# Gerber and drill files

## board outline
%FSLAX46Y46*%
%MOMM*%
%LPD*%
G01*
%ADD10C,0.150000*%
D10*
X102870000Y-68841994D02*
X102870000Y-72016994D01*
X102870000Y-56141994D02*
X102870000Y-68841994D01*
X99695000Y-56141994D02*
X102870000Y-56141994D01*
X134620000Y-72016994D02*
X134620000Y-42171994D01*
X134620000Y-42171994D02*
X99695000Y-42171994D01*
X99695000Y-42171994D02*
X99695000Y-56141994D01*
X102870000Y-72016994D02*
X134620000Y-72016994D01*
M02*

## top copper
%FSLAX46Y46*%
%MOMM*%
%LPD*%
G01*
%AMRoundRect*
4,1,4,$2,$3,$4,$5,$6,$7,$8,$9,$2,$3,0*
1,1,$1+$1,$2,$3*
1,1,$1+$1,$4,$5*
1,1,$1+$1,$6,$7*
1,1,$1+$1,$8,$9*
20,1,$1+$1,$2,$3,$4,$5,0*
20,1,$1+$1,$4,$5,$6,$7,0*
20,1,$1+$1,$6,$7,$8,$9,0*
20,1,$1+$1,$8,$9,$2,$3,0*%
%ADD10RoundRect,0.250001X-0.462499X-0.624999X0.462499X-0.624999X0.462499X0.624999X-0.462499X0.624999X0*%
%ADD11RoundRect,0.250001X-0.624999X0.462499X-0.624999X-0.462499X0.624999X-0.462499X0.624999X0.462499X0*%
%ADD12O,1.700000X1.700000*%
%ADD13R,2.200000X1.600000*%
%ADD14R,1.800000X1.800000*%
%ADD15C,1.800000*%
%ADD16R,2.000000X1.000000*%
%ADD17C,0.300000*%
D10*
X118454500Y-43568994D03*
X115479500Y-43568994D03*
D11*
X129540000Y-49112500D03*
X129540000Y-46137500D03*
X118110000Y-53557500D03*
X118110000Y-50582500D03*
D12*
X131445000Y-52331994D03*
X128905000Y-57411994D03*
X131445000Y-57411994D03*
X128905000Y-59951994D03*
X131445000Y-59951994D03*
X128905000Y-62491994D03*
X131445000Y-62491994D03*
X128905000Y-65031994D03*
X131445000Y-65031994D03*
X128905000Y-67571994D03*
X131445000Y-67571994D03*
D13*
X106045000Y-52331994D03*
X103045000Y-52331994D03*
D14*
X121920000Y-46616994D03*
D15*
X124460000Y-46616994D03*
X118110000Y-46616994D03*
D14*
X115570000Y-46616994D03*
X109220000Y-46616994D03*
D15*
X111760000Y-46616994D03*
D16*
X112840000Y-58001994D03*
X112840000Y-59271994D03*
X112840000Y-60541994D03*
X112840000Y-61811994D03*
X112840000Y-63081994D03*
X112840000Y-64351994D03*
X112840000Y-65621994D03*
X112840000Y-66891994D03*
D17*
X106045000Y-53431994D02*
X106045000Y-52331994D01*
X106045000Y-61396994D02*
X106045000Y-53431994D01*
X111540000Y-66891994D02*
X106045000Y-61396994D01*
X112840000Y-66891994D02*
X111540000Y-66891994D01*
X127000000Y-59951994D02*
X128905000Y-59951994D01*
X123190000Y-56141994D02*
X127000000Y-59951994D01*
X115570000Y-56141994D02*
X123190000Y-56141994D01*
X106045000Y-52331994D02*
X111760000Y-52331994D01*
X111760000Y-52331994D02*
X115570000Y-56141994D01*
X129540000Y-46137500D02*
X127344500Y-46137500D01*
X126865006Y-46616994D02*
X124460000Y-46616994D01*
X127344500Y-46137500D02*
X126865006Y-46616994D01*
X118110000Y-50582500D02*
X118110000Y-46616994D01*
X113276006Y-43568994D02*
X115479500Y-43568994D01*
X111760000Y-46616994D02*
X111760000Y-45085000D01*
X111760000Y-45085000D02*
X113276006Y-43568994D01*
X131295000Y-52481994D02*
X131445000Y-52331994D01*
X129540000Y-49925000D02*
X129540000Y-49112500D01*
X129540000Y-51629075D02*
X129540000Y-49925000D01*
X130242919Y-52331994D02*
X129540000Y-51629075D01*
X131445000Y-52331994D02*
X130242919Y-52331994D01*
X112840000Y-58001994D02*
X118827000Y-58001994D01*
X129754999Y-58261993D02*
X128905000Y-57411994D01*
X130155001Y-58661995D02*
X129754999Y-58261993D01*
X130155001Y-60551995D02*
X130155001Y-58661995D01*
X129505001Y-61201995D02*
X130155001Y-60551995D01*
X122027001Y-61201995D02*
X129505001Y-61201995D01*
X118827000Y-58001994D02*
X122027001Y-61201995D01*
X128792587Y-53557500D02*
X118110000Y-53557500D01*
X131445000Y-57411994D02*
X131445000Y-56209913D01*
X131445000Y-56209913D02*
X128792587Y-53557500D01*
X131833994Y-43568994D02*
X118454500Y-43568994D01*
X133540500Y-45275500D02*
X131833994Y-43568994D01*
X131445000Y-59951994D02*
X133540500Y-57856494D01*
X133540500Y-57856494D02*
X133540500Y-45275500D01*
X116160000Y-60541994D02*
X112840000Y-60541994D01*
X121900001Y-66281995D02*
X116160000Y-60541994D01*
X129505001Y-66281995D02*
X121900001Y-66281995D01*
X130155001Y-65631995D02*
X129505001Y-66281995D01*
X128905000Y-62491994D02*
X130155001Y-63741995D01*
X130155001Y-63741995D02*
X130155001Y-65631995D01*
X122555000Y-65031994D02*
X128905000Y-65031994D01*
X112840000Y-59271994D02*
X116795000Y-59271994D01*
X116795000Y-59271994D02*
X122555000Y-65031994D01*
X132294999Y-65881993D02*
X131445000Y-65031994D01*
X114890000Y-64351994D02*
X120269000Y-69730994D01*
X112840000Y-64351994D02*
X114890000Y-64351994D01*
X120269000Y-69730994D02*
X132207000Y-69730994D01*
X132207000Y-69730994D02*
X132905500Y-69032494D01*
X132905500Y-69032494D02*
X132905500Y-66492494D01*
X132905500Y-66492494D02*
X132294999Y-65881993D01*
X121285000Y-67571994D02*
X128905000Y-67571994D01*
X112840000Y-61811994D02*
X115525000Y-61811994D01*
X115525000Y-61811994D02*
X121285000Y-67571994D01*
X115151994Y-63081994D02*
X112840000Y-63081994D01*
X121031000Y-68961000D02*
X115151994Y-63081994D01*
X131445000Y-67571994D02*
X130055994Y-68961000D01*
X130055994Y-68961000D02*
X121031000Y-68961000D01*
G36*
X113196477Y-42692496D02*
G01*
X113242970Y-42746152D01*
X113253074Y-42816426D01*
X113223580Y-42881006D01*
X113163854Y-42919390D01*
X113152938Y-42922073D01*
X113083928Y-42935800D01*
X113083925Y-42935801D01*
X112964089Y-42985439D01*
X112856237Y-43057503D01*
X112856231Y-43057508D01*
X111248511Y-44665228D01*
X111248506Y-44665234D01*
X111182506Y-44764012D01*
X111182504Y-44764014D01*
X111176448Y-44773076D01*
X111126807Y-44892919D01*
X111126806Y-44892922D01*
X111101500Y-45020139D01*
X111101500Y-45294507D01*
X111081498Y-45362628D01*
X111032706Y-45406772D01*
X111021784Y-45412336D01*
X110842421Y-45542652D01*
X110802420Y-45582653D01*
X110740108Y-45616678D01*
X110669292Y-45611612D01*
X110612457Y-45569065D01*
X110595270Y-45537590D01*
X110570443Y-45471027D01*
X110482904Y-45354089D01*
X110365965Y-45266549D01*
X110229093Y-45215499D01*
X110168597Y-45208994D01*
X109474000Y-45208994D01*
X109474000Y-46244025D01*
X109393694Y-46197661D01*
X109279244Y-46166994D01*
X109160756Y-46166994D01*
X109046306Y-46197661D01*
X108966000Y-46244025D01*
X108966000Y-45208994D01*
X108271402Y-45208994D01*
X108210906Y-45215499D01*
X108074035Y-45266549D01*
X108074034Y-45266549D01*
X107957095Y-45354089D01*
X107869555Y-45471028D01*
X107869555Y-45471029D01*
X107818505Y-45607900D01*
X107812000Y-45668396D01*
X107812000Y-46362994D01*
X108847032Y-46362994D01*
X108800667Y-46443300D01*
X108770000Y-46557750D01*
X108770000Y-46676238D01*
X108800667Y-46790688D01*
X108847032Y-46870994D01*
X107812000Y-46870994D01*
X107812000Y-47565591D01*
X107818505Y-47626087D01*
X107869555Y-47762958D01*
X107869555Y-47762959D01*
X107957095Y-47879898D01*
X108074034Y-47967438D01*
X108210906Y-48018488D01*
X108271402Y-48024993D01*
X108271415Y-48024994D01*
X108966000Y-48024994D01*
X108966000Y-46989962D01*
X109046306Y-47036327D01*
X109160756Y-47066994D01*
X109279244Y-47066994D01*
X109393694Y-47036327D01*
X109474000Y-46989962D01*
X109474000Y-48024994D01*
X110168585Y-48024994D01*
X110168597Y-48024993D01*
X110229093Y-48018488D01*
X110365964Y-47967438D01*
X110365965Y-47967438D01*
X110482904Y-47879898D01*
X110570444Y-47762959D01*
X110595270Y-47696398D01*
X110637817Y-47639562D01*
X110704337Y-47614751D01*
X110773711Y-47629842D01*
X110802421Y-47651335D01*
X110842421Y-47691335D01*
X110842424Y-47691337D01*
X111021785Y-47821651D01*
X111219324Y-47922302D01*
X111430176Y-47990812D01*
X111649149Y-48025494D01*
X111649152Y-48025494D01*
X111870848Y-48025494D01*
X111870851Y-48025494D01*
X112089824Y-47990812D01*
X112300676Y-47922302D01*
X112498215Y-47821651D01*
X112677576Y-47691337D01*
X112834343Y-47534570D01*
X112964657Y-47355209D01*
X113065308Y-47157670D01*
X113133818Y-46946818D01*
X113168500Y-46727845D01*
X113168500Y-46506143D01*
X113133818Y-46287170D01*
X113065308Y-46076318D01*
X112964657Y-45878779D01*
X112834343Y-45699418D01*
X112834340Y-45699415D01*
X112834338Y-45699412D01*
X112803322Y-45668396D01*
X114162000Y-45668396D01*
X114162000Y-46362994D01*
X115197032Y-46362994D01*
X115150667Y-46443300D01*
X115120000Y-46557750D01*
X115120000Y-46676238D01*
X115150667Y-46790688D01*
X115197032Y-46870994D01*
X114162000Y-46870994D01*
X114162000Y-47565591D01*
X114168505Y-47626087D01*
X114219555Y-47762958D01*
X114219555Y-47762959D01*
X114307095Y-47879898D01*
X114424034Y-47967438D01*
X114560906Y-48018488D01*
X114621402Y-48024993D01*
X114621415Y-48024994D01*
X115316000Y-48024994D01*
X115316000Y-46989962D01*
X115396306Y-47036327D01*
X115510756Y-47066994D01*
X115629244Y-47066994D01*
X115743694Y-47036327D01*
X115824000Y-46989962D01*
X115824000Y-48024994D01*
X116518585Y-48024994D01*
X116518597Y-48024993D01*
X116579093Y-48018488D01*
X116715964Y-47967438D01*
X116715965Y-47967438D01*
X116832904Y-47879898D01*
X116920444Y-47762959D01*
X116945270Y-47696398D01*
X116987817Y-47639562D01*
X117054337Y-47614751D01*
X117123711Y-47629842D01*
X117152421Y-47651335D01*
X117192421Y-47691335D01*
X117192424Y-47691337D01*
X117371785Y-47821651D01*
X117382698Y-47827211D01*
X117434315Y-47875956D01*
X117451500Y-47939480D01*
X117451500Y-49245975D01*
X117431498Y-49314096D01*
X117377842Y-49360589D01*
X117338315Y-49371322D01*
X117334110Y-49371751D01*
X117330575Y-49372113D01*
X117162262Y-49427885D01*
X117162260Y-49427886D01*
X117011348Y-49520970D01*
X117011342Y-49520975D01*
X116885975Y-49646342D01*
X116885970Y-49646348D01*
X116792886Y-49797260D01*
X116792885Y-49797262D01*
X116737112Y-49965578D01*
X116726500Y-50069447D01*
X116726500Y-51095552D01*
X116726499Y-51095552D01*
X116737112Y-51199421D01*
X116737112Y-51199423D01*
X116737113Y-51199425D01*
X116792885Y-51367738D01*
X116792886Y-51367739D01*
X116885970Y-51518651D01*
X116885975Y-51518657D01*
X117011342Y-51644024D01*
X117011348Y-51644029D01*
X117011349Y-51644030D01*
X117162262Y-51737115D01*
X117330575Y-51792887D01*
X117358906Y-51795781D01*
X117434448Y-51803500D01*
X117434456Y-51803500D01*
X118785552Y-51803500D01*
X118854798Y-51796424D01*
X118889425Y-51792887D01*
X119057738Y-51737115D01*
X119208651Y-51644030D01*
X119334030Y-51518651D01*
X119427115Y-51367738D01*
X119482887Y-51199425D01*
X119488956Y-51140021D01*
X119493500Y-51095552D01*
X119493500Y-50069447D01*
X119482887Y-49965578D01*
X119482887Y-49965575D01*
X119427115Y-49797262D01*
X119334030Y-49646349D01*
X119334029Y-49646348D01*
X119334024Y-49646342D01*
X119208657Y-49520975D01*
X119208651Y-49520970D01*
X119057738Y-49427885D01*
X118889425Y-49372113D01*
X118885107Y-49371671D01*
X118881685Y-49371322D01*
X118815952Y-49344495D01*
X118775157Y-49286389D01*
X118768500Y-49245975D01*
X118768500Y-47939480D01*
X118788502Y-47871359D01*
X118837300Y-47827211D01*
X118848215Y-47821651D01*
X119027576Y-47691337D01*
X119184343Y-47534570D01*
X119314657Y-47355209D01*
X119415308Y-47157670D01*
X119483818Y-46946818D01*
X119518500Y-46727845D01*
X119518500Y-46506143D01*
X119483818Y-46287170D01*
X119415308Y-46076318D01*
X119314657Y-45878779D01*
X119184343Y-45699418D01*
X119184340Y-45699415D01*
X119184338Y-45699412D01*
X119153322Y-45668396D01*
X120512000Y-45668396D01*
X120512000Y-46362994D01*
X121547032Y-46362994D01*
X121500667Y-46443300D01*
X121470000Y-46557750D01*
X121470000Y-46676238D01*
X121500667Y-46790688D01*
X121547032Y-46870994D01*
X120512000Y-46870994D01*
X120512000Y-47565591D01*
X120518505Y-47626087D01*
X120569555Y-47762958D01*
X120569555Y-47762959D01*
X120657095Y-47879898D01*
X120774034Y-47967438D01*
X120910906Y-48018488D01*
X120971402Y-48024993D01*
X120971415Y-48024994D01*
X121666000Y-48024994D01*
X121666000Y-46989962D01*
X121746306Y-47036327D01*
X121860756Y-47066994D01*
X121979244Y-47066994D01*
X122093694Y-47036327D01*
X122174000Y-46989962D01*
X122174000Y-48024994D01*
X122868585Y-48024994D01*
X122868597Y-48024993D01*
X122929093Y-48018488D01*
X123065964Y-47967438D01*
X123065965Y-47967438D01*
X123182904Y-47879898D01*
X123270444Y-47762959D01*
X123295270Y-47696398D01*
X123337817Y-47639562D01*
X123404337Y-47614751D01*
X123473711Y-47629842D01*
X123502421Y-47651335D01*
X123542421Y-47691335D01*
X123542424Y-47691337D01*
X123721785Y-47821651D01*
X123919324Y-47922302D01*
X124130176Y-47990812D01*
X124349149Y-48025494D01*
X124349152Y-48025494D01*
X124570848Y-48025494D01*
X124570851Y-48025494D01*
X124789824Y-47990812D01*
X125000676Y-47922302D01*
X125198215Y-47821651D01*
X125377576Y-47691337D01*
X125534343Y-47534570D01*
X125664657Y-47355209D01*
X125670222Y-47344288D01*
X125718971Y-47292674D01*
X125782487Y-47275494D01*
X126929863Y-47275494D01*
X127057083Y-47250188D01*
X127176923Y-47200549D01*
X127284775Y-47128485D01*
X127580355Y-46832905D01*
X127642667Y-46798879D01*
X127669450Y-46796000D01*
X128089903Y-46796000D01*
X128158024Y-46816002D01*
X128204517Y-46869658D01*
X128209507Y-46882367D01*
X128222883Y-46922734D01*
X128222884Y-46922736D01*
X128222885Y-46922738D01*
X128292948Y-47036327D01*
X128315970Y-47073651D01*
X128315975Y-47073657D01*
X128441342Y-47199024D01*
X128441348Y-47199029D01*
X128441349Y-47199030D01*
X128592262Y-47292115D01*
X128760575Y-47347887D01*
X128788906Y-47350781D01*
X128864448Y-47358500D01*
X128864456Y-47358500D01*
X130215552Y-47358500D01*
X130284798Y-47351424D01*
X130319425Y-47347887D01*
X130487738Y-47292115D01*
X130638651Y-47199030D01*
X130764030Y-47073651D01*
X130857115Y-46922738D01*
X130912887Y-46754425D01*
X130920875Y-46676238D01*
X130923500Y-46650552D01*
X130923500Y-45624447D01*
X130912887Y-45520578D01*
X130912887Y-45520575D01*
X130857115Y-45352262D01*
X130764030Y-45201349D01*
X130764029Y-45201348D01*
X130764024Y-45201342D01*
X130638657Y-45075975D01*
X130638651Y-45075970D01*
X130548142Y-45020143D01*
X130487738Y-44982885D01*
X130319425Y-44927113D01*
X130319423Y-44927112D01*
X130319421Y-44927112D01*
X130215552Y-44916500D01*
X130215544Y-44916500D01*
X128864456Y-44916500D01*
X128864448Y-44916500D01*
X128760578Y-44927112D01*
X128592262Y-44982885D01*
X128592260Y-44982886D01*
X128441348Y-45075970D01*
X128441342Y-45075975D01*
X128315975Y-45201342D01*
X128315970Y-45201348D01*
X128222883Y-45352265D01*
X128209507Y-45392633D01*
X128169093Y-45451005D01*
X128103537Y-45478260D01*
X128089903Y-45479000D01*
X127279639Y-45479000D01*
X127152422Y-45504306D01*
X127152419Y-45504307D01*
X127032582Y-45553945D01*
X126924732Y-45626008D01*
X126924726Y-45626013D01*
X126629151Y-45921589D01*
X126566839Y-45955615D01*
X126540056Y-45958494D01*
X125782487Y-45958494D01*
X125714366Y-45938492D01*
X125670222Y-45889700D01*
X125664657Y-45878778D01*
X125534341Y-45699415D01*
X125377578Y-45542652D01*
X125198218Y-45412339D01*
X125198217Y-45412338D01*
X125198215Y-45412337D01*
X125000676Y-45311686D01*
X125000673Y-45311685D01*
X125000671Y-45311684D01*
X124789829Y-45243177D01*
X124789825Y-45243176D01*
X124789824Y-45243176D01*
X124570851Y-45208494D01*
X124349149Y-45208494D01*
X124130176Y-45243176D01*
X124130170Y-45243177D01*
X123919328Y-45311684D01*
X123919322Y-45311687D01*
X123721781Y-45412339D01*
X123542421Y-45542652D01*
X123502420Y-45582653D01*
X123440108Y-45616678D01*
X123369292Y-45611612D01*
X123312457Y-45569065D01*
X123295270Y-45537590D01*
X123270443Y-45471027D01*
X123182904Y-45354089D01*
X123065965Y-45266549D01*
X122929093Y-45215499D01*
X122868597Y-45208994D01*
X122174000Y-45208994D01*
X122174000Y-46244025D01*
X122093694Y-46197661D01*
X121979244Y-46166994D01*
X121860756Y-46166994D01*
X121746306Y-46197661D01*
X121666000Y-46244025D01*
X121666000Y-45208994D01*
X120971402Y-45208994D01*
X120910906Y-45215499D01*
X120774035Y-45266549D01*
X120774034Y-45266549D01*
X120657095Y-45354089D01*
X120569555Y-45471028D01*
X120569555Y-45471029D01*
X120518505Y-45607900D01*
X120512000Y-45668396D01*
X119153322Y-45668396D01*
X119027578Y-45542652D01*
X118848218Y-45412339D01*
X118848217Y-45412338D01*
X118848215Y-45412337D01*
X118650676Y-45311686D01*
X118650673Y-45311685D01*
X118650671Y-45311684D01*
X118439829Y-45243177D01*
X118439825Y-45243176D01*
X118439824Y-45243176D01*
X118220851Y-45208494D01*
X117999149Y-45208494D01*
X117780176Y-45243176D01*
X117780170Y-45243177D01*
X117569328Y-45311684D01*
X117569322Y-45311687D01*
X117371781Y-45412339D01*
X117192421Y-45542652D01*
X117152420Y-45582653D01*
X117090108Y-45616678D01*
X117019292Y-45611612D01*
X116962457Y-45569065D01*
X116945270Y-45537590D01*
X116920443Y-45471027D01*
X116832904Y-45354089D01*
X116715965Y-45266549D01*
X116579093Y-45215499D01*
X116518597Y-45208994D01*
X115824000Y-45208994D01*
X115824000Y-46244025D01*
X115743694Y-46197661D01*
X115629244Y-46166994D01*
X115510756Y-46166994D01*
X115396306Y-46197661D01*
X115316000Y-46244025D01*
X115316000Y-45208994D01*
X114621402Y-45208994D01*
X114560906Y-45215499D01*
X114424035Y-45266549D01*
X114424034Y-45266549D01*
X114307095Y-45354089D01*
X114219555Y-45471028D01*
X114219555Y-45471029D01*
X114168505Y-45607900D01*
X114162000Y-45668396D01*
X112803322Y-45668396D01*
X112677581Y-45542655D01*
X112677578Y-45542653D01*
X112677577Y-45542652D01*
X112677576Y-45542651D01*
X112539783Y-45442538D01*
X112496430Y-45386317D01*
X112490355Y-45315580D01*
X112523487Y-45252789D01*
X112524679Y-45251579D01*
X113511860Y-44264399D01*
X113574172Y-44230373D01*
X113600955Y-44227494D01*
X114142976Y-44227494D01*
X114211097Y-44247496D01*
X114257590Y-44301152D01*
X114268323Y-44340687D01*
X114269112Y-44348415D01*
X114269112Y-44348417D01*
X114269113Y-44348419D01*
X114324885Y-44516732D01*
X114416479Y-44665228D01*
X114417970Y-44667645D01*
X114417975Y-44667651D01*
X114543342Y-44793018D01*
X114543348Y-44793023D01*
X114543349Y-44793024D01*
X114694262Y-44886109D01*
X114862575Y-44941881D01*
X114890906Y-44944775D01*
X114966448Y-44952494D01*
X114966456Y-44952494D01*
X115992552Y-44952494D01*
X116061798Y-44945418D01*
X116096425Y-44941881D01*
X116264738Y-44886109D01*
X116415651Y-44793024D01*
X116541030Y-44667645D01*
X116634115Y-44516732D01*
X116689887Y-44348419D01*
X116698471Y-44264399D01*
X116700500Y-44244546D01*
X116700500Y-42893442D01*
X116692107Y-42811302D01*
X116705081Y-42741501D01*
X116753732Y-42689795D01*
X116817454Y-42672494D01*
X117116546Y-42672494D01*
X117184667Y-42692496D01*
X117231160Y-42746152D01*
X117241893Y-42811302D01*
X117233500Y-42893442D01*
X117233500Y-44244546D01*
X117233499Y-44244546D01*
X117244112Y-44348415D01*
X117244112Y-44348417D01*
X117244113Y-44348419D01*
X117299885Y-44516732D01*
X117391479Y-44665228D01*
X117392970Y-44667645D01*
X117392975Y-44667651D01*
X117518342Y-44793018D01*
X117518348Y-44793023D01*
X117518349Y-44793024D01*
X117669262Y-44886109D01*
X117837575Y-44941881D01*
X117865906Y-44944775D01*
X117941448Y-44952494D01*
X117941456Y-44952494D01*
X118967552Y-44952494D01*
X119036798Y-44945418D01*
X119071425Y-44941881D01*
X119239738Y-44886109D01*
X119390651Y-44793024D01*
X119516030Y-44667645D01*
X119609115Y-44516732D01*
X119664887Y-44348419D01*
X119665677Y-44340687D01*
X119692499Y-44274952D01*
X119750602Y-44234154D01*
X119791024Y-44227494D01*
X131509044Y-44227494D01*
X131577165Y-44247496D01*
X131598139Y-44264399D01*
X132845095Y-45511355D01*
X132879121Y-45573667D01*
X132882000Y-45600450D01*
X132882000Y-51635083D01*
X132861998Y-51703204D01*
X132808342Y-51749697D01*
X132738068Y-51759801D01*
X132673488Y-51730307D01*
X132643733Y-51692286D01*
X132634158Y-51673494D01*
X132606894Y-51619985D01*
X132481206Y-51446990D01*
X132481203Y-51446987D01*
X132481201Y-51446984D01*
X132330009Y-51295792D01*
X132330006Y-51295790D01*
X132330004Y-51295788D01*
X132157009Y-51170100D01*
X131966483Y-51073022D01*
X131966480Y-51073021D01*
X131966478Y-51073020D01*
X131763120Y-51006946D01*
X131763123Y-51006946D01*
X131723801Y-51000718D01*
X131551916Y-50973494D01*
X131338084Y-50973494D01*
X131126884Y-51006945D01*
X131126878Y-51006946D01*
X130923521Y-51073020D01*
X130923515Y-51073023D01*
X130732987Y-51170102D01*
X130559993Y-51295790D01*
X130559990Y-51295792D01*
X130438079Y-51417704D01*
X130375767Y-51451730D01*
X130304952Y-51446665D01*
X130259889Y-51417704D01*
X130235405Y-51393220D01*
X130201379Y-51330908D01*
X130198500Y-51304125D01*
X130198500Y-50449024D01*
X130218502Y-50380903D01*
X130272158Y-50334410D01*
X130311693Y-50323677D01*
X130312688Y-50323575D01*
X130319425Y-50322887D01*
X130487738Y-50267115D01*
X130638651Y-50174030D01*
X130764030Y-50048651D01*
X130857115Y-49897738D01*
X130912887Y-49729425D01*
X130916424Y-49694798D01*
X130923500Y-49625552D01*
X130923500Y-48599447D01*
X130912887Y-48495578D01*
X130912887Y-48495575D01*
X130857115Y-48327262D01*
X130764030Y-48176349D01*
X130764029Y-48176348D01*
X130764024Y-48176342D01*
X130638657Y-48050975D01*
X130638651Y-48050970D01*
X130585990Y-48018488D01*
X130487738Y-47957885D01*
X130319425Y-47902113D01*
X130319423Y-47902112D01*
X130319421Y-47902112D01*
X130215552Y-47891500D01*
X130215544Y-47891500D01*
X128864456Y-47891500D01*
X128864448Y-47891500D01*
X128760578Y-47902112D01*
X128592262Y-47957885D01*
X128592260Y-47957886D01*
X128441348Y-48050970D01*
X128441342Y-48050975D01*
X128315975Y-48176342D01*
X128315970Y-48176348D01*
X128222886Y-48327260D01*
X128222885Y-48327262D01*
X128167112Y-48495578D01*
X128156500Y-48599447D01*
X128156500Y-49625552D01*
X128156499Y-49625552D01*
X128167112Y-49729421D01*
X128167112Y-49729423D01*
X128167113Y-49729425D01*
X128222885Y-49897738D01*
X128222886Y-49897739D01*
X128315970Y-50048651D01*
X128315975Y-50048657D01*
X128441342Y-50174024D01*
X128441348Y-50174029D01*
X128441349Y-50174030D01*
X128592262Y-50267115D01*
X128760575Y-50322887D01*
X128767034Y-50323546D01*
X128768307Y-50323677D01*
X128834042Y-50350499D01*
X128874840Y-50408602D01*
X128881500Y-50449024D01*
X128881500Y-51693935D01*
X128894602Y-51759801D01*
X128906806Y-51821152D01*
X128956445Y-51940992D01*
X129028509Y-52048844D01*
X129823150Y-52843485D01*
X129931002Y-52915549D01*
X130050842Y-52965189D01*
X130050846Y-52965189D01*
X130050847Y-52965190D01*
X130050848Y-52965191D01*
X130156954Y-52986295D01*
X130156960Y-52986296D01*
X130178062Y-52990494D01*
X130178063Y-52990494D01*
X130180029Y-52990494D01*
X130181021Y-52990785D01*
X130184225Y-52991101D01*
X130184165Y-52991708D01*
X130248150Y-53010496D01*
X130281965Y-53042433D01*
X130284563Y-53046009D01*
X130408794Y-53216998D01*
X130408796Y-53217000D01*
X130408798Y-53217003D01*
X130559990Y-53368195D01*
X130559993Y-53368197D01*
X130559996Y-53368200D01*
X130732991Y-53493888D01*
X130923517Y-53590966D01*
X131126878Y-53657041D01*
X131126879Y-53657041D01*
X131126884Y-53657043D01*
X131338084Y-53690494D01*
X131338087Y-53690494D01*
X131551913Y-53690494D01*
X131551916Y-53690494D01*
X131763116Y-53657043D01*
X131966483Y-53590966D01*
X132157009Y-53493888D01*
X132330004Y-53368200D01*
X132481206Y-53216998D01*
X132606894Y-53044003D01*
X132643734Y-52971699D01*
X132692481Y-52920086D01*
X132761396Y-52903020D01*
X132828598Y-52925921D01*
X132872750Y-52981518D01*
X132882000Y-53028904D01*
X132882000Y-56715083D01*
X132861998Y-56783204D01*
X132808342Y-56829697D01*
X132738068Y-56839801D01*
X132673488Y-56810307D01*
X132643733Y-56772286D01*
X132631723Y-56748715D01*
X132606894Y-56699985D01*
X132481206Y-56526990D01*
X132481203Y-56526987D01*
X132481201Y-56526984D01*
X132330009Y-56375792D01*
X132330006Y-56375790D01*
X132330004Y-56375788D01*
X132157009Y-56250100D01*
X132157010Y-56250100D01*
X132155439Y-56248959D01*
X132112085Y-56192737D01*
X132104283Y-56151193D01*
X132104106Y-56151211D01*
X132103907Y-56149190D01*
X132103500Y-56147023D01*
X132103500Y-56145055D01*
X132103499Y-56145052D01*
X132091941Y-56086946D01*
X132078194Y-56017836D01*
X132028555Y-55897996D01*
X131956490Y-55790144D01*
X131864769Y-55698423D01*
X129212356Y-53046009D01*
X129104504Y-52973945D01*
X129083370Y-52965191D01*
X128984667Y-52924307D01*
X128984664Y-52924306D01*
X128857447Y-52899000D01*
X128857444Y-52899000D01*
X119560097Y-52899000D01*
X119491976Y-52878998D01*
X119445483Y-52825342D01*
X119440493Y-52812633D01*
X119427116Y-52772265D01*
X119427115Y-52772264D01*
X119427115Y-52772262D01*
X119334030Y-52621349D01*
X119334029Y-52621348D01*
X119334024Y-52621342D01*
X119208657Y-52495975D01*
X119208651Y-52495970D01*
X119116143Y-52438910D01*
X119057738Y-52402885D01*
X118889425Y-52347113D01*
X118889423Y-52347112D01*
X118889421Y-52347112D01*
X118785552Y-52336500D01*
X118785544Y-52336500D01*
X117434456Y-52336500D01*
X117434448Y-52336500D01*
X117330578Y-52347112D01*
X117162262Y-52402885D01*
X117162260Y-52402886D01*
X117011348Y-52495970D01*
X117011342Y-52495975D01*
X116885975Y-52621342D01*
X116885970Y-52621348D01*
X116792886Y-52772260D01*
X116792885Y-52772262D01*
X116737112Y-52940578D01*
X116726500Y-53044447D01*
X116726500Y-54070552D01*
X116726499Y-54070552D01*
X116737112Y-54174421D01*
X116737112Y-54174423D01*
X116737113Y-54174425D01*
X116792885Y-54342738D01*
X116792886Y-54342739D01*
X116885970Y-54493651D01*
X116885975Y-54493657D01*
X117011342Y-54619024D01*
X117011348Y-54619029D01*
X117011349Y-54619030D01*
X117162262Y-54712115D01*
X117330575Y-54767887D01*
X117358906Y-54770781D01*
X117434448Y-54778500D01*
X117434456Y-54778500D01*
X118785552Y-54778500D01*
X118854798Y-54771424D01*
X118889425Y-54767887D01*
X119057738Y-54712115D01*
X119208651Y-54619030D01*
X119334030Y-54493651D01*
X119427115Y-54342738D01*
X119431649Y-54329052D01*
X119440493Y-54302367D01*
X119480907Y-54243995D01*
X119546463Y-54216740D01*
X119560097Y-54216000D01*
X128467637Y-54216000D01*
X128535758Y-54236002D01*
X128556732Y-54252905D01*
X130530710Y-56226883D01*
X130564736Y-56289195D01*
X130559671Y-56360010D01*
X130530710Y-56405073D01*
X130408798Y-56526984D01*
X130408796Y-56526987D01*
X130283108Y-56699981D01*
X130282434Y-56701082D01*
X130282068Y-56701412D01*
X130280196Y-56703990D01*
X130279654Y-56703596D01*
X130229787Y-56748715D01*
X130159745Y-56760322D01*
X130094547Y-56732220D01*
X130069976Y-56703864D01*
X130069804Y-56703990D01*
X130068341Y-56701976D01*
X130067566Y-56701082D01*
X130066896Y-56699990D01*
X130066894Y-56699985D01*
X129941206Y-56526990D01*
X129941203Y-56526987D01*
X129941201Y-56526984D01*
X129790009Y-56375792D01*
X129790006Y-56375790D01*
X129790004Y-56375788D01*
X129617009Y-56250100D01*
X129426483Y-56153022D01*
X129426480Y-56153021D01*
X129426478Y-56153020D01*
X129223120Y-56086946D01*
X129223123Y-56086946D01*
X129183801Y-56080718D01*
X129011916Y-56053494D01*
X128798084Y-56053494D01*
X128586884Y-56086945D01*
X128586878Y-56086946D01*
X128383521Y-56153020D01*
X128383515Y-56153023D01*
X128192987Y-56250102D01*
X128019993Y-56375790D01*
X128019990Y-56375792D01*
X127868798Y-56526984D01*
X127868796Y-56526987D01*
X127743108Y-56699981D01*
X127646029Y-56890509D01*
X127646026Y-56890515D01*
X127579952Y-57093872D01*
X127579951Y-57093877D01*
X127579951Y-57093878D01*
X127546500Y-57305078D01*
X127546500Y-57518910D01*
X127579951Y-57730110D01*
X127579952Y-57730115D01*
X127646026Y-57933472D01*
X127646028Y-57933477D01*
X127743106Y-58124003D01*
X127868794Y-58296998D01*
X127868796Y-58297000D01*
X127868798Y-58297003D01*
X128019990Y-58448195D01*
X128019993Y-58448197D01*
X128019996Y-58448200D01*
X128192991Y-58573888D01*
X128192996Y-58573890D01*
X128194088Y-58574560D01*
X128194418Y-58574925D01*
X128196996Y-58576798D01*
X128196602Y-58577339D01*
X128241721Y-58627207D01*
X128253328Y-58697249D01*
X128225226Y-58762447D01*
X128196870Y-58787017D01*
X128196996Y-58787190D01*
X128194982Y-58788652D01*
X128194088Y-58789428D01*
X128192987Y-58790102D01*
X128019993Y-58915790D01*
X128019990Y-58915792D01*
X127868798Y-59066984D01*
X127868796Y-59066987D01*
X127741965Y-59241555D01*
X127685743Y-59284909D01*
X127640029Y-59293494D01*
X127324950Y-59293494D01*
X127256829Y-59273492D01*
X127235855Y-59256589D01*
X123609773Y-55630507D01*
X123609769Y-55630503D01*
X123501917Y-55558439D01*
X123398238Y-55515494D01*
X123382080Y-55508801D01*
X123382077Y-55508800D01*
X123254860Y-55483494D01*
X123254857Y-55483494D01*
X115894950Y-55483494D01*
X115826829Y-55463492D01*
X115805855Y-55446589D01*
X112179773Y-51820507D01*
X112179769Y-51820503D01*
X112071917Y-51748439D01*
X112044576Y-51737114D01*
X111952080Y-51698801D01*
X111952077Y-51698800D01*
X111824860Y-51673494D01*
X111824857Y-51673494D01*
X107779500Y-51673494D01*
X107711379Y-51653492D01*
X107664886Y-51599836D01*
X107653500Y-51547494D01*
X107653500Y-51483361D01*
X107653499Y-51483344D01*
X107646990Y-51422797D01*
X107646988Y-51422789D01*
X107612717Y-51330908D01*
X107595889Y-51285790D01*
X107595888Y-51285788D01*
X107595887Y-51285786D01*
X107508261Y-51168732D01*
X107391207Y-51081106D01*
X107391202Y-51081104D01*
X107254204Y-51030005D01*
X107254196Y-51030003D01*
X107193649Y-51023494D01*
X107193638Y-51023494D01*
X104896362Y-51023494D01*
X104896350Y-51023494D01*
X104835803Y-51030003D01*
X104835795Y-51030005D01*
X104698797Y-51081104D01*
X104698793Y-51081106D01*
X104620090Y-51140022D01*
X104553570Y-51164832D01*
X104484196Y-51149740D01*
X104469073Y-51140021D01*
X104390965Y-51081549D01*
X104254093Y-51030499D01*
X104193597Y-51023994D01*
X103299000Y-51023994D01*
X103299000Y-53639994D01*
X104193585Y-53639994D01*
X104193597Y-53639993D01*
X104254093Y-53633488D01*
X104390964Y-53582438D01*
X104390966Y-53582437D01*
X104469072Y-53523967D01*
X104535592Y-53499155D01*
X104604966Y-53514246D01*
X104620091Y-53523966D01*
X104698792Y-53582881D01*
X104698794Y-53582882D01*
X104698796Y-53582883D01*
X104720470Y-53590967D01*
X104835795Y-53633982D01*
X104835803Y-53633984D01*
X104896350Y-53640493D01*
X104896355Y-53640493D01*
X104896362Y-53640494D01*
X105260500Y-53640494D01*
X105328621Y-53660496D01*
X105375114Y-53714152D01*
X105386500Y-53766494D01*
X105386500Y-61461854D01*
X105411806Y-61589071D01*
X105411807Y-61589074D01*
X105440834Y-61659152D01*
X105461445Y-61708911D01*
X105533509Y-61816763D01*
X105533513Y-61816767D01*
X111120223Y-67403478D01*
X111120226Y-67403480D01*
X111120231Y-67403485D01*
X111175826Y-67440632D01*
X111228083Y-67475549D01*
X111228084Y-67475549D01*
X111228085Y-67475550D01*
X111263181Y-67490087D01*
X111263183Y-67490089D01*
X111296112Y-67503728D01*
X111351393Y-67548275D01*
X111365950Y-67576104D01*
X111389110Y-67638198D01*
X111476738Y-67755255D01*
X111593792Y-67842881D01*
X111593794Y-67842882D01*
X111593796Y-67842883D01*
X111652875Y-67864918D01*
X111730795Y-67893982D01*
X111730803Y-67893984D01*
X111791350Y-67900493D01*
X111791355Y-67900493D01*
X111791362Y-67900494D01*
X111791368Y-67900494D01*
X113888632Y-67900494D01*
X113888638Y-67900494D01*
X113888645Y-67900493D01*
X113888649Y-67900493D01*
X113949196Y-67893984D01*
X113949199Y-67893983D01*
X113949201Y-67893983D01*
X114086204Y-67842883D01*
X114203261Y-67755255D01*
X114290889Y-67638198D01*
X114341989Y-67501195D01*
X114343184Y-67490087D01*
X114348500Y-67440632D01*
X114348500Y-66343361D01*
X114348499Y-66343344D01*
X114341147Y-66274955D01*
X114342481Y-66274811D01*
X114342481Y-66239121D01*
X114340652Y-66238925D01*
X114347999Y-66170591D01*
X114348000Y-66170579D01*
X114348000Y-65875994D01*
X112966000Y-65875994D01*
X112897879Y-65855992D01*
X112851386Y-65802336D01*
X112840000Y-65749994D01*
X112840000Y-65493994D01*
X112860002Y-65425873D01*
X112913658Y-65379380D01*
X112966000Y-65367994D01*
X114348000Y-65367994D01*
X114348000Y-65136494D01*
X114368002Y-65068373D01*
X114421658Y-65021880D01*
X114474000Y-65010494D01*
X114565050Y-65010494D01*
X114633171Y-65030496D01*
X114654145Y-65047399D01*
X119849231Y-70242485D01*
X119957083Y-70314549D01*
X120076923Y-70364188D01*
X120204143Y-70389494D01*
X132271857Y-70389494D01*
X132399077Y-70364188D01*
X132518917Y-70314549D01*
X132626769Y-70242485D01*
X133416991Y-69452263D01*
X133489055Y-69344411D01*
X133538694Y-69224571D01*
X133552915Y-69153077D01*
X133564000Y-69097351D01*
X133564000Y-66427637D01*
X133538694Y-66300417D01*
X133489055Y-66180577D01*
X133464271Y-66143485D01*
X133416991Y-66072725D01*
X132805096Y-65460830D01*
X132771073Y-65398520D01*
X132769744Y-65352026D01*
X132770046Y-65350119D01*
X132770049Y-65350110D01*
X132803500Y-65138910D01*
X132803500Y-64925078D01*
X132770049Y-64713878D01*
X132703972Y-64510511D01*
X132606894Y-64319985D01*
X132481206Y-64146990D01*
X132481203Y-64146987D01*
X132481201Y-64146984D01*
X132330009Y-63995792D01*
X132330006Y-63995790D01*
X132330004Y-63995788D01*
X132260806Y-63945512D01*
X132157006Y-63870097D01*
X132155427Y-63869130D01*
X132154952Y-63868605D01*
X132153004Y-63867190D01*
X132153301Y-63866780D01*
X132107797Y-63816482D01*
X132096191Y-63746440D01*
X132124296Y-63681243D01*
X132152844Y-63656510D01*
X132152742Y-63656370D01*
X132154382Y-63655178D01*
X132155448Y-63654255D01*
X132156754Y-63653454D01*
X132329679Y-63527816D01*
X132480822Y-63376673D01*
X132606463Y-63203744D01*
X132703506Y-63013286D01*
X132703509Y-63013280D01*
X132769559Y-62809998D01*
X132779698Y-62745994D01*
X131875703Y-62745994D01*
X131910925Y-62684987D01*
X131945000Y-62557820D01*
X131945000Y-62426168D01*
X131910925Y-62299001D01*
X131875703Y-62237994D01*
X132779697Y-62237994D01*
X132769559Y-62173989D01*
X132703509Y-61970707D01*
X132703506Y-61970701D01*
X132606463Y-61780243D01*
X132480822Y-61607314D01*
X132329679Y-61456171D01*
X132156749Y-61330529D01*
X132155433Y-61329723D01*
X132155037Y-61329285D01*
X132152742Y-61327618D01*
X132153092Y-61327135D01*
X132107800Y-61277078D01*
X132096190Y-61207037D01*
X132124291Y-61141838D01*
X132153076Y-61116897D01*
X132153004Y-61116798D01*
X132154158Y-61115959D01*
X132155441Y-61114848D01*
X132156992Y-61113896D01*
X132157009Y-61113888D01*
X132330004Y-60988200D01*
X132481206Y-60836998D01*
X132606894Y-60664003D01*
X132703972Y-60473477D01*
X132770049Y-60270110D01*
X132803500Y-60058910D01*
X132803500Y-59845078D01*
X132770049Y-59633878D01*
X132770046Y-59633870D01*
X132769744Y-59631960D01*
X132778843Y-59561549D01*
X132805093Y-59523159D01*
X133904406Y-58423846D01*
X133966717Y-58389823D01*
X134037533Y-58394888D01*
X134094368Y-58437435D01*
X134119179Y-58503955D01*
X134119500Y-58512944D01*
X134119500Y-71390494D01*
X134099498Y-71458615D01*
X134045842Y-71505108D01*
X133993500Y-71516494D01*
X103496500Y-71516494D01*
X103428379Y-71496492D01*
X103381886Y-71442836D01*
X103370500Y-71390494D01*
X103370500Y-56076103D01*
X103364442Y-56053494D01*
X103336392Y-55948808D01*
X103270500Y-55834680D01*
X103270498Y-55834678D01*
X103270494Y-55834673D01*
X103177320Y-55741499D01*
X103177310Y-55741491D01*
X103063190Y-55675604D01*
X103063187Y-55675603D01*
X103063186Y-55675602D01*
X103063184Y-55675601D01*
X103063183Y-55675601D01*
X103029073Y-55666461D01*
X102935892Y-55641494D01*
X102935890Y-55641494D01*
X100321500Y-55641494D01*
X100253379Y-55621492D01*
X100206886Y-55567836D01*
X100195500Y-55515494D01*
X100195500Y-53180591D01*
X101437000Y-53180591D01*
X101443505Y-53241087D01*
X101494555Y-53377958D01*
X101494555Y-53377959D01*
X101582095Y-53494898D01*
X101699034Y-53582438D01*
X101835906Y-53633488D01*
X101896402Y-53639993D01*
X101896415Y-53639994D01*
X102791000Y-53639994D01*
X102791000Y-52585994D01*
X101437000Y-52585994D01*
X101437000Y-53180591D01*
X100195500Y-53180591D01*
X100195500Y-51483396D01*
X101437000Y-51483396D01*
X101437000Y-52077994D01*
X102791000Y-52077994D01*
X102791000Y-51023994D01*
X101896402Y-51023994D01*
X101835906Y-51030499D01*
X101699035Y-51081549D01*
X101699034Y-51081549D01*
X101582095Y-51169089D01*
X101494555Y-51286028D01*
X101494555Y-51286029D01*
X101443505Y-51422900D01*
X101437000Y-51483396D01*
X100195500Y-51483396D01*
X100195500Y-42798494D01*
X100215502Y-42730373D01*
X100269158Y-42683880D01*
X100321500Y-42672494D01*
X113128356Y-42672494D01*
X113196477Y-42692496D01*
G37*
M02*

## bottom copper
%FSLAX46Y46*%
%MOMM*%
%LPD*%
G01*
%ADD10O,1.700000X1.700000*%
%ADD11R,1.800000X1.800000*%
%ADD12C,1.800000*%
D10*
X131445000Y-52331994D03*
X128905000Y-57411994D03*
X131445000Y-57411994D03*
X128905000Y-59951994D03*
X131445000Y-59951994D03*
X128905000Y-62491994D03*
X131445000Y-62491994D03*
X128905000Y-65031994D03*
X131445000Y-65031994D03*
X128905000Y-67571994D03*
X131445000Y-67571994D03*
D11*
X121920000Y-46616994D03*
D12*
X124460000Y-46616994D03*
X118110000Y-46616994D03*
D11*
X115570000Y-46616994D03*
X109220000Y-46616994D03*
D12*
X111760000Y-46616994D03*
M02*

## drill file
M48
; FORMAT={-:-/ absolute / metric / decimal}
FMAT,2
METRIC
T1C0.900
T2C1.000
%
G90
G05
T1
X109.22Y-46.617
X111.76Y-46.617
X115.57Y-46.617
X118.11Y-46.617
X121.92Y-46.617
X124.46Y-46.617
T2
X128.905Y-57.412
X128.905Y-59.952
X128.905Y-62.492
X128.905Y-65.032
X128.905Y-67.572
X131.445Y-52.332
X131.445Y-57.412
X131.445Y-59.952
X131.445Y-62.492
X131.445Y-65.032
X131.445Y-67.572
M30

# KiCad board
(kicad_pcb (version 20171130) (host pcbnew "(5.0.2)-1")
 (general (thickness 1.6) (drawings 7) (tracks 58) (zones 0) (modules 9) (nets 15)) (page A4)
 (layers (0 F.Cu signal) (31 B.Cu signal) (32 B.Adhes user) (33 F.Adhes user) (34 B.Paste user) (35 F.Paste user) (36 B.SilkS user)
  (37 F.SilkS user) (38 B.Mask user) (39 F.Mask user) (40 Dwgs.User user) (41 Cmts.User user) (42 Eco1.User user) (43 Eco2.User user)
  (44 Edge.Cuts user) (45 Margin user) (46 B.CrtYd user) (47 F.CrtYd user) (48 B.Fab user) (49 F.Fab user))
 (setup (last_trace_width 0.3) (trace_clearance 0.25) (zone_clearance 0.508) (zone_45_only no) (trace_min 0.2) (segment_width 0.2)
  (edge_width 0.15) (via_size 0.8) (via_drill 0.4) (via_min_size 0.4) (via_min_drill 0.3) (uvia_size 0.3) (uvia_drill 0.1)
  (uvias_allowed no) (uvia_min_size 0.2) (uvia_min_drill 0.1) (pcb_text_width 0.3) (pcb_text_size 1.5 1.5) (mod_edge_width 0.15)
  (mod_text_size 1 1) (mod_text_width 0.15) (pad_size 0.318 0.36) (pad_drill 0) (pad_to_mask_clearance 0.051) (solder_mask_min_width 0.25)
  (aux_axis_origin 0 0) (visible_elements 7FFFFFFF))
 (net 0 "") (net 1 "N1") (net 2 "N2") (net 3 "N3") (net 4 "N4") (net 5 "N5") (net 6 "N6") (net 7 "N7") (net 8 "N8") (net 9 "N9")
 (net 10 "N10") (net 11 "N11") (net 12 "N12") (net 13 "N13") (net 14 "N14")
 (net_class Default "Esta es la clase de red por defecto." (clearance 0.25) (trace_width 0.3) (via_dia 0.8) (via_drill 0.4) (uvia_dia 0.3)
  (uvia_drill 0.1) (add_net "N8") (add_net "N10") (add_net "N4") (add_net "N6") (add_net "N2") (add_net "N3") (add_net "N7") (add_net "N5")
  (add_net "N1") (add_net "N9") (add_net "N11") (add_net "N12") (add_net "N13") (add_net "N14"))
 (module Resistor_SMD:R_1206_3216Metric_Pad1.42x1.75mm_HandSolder (layer F.Cu) (at 116.967 43.568994)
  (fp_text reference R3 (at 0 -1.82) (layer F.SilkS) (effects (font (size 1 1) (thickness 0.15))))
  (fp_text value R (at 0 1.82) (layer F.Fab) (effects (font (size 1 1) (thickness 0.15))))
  (pad 2 smd roundrect (at 1.4875 0) (size 1.425 1.75) (layers F.Cu F.Paste F.Mask) (roundrect_rratio 0.175439) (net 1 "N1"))
  (pad 1 smd roundrect (at -1.4875 0) (size 1.425 1.75) (layers F.Cu F.Paste F.Mask) (roundrect_rratio 0.175439) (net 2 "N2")))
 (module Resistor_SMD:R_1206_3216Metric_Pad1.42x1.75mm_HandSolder (layer F.Cu) (at 129.54 47.625 270)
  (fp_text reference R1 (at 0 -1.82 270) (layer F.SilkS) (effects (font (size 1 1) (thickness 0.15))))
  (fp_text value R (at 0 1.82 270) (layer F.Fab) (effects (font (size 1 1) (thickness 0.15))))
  (pad 2 smd roundrect (at 1.4875 0 270) (size 1.425 1.75) (layers F.Cu F.Paste F.Mask) (roundrect_rratio 0.175439) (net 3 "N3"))
  (pad 1 smd roundrect (at -1.4875 0 270) (size 1.425 1.75) (layers F.Cu F.Paste F.Mask) (roundrect_rratio 0.175439) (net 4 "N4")))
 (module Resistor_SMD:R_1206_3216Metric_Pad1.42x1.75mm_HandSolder (layer F.Cu) (at 118.11 52.07 270)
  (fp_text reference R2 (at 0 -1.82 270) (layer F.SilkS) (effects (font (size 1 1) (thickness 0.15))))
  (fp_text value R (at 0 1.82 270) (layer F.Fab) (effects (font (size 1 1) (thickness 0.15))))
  (pad 2 smd roundrect (at 1.4875 0 270) (size 1.425 1.75) (layers F.Cu F.Paste F.Mask) (roundrect_rratio 0.175439) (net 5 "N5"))
  (pad 1 smd roundrect (at -1.4875 0 270) (size 1.425 1.75) (layers F.Cu F.Paste F.Mask) (roundrect_rratio 0.175439) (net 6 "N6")))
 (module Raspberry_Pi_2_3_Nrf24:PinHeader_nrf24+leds (layer F.Cu) (at 129.794 59.799594)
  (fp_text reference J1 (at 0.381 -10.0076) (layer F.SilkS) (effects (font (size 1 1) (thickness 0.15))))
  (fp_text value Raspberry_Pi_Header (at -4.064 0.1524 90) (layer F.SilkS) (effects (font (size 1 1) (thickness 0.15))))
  (pad 12 thru_hole oval (at 1.651 -7.4676) (size 1.7 1.7) (drill 1) (layers *.Cu *.Mask) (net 3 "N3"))
  (pad 15 thru_hole oval (at -0.889 -2.3876) (size 1.7 1.7) (drill 1) (layers *.Cu *.Mask) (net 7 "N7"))
  (pad 16 thru_hole oval (at 1.651 -2.3876) (size 1.7 1.7) (drill 1) (layers *.Cu *.Mask) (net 5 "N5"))
  (pad 17 thru_hole oval (at -0.889 0.1524) (size 1.7 1.7) (drill 1) (layers *.Cu *.Mask) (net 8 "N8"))
  (pad 18 thru_hole oval (at 1.651 0.1524) (size 1.7 1.7) (drill 1) (layers *.Cu *.Mask) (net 1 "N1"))
  (pad 19 thru_hole oval (at -0.889 2.6924) (size 1.7 1.7) (drill 1) (layers *.Cu *.Mask) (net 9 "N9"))
  (pad 20 thru_hole oval (at 1.651 2.6924) (size 1.7 1.7) (drill 1) (layers *.Cu *.Mask) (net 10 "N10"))
  (pad 21 thru_hole oval (at -0.889 5.2324) (size 1.7 1.7) (drill 1) (layers *.Cu *.Mask) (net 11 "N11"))
  (pad 22 thru_hole oval (at 1.651 5.2324) (size 1.7 1.7) (drill 1) (layers *.Cu *.Mask) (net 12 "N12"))
  (pad 23 thru_hole oval (at -0.889 7.7724) (size 1.7 1.7) (drill 1) (layers *.Cu *.Mask) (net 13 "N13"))
  (pad 24 thru_hole oval (at 1.651 7.7724) (size 1.7 1.7) (drill 1) (layers *.Cu *.Mask) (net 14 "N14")))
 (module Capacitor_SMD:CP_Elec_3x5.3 (layer F.Cu) (at 104.545 52.331994 180)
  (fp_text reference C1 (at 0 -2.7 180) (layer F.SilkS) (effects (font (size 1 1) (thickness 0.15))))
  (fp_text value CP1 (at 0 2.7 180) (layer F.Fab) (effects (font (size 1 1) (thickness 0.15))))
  (pad 1 smd rect (at -1.5 0 180) (size 2.2 1.6) (layers F.Cu F.Paste F.Mask) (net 8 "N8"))
  (pad 2 smd rect (at 1.5 0 180) (size 2.2 1.6) (layers F.Cu F.Paste F.Mask) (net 10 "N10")))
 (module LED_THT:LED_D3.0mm (layer F.Cu) (at 121.92 46.616994)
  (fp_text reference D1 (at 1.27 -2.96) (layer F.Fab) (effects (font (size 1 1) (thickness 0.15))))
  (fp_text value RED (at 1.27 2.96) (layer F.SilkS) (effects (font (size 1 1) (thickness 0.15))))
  (pad 1 thru_hole rect (at 0 0) (size 1.8 1.8) (drill 0.9) (layers *.Cu *.Mask) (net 10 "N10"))
  (pad 2 thru_hole circle (at 2.54 0) (size 1.8 1.8) (drill 0.9) (layers *.Cu *.Mask) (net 4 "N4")))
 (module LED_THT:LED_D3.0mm (layer F.Cu) (at 115.57 46.616994)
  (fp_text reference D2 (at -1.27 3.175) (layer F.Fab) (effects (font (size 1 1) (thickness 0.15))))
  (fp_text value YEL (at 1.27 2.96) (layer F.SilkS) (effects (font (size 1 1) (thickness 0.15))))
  (pad 2 thru_hole circle (at 2.54 0) (size 1.8 1.8) (drill 0.9) (layers *.Cu *.Mask) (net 6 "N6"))
  (pad 1 thru_hole rect (at 0 0) (size 1.8 1.8) (drill 0.9) (layers *.Cu *.Mask) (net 10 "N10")))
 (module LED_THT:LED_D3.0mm (layer F.Cu) (at 109.22 46.616994)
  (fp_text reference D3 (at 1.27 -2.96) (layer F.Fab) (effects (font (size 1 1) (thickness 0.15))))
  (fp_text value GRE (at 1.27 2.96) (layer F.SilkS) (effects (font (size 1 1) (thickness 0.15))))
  (pad 1 thru_hole rect (at 0 0) (size 1.8 1.8) (drill 0.9) (layers *.Cu *.Mask) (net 10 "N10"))
  (pad 2 thru_hole circle (at 2.54 0) (size 1.8 1.8) (drill 0.9) (layers *.Cu *.Mask) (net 2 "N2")))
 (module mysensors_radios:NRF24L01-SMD (layer F.Cu) (at 104.14 62.491994 90)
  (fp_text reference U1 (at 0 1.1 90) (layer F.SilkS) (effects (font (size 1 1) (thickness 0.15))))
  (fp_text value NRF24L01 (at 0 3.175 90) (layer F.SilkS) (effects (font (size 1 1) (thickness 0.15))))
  (pad 8 smd rect (at 4.49 8.7 90) (size 1 2) (layers F.Cu F.Paste F.Mask) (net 7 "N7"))
  (pad 7 smd rect (at 3.22 8.7 90) (size 1 2) (layers F.Cu F.Paste F.Mask) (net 11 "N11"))
  (pad 6 smd rect (at 1.95 8.7 90) (size 1 2) (layers F.Cu F.Paste F.Mask) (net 9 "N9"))
  (pad 5 smd rect (at 0.68 8.7 90) (size 1 2) (layers F.Cu F.Paste F.Mask) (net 13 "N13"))
  (pad 4 smd rect (at -0.59 8.7 90) (size 1 2) (layers F.Cu F.Paste F.Mask) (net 14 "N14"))
  (pad 3 smd rect (at -1.86 8.7 90) (size 1 2) (layers F.Cu F.Paste F.Mask) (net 12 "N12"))
  (pad 1 smd rect (at -3.13 8.7 90) (size 1 2) (layers F.Cu F.Paste F.Mask) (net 10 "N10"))
  (pad 2 smd rect (at -4.4 8.7 90) (size 1 2) (layers F.Cu F.Paste F.Mask) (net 8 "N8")))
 (gr_line (start 102.87 68.841994) (end 102.87 72.016994) (layer Edge.Cuts) (width 0.15))
 (gr_line (start 102.87 56.141994) (end 102.87 68.841994) (layer Edge.Cuts) (width 0.15))
 (gr_line (start 99.695 56.141994) (end 102.87 56.141994) (layer Edge.Cuts) (width 0.15))
 (gr_line (start 134.62 72.016994) (end 134.62 42.171994) (layer Edge.Cuts) (width 0.15))
 (gr_line (start 134.62 42.171994) (end 99.695 42.171994) (layer Edge.Cuts) (width 0.15))
 (gr_line (start 99.695 42.171994) (end 99.695 56.141994) (layer Edge.Cuts) (width 0.15))
 (gr_line (start 102.87 72.016994) (end 134.62 72.016994) (layer Edge.Cuts) (width 0.15))
 (segment (start 106.045 53.431994) (end 106.045 52.331994) (width 0.3) (layer F.Cu) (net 8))
 (segment (start 106.045 61.396994) (end 106.045 53.431994) (width 0.3) (layer F.Cu) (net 8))
 (segment (start 111.54 66.891994) (end 106.045 61.396994) (width 0.3) (layer F.Cu) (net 8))
 (segment (start 112.84 66.891994) (end 111.54 66.891994) (width 0.3) (layer F.Cu) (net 8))
 (segment (start 127 59.951994) (end 128.905 59.951994) (width 0.3) (layer F.Cu) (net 8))
 (segment (start 123.19 56.141994) (end 127 59.951994) (width 0.3) (layer F.Cu) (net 8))
 (segment (start 115.57 56.141994) (end 123.19 56.141994) (width 0.3) (layer F.Cu) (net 8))
 (segment (start 106.045 52.331994) (end 111.76 52.331994) (width 0.3) (layer F.Cu) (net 8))
 (segment (start 111.76 52.331994) (end 115.57 56.141994) (width 0.3) (layer F.Cu) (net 8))
 (segment (start 129.54 46.1375) (end 127.3445 46.1375) (width 0.3) (layer F.Cu) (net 4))
 (segment (start 126.865006 46.616994) (end 124.46 46.616994) (width 0.3) (layer F.Cu) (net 4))
 (segment (start 127.3445 46.1375) (end 126.865006 46.616994) (width 0.3) (layer F.Cu) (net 4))
 (segment (start 118.11 50.5825) (end 118.11 46.616994) (width 0.3) (layer F.Cu) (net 6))
 (segment (start 113.276006 43.568994) (end 115.4795 43.568994) (width 0.3) (layer F.Cu) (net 2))
 (segment (start 111.76 46.616994) (end 111.76 45.085) (width 0.3) (layer F.Cu) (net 2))
 (segment (start 111.76 45.085) (end 113.276006 43.568994) (width 0.3) (layer F.Cu) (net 2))
 (segment (start 131.295 52.481994) (end 131.445 52.331994) (width 0.3) (layer F.Cu) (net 3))
 (segment (start 129.54 49.925) (end 129.54 49.1125) (width 0.3) (layer F.Cu) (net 3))
 (segment (start 129.54 51.629075) (end 129.54 49.925) (width 0.3) (layer F.Cu) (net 3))
 (segment (start 130.242919 52.331994) (end 129.54 51.629075) (width 0.3) (layer F.Cu) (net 3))
 (segment (start 131.445 52.331994) (end 130.242919 52.331994) (width 0.3) (layer F.Cu) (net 3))
 (segment (start 112.84 58.001994) (end 118.827 58.001994) (width 0.3) (layer F.Cu) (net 7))
 (segment (start 129.754999 58.261993) (end 128.905 57.411994) (width 0.3) (layer F.Cu) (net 7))
 (segment (start 130.155001 58.661995) (end 129.754999 58.261993) (width 0.3) (layer F.Cu) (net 7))
 (segment (start 130.155001 60.551995) (end 130.155001 58.661995) (width 0.3) (layer F.Cu) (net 7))
 (segment (start 129.505001 61.201995) (end 130.155001 60.551995) (width 0.3) (layer F.Cu) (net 7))
 (segment (start 122.027001 61.201995) (end 129.505001 61.201995) (width 0.3) (layer F.Cu) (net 7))
 (segment (start 118.827 58.001994) (end 122.027001 61.201995) (width 0.3) (layer F.Cu) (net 7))
 (segment (start 128.792587 53.5575) (end 118.11 53.5575) (width 0.3) (layer F.Cu) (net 5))
 (segment (start 131.445 57.411994) (end 131.445 56.209913) (width 0.3) (layer F.Cu) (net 5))
 (segment (start 131.445 56.209913) (end 128.792587 53.5575) (width 0.3) (layer F.Cu) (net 5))
 (segment (start 131.833994 43.568994) (end 118.4545 43.568994) (width 0.3) (layer F.Cu) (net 1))
 (segment (start 133.5405 45.2755) (end 131.833994 43.568994) (width 0.3) (layer F.Cu) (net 1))
 (segment (start 131.445 59.951994) (end 133.5405 57.856494) (width 0.3) (layer F.Cu) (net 1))
 (segment (start 133.5405 57.856494) (end 133.5405 45.2755) (width 0.3) (layer F.Cu) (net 1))
 (segment (start 116.16 60.541994) (end 112.84 60.541994) (width 0.3) (layer F.Cu) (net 9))
 (segment (start 121.900001 66.281995) (end 116.16 60.541994) (width 0.3) (layer F.Cu) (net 9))
 (segment (start 129.505001 66.281995) (end 121.900001 66.281995) (width 0.3) (layer F.Cu) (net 9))
 (segment (start 130.155001 65.631995) (end 129.505001 66.281995) (width 0.3) (layer F.Cu) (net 9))
 (segment (start 128.905 62.491994) (end 130.155001 63.741995) (width 0.3) (layer F.Cu) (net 9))
 (segment (start 130.155001 63.741995) (end 130.155001 65.631995) (width 0.3) (layer F.Cu) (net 9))
 (segment (start 122.555 65.031994) (end 128.905 65.031994) (width 0.3) (layer F.Cu) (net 11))
 (segment (start 112.84 59.271994) (end 116.795 59.271994) (width 0.3) (layer F.Cu) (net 11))
 (segment (start 116.795 59.271994) (end 122.555 65.031994) (width 0.3) (layer F.Cu) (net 11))
 (segment (start 132.294999 65.881993) (end 131.445 65.031994) (width 0.3) (layer F.Cu) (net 12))
 (segment (start 114.89 64.351994) (end 120.269 69.730994) (width 0.3) (layer F.Cu) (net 12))
 (segment (start 112.84 64.351994) (end 114.89 64.351994) (width 0.3) (layer F.Cu) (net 12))
 (segment (start 120.269 69.730994) (end 132.207 69.730994) (width 0.3) (layer F.Cu) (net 12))
 (segment (start 132.207 69.730994) (end 132.9055 69.032494) (width 0.3) (layer F.Cu) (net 12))
 (segment (start 132.9055 69.032494) (end 132.9055 66.492494) (width 0.3) (layer F.Cu) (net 12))
 (segment (start 132.9055 66.492494) (end 132.294999 65.881993) (width 0.3) (layer F.Cu) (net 12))
 (segment (start 121.285 67.571994) (end 128.905 67.571994) (width 0.3) (layer F.Cu) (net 13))
 (segment (start 112.84 61.811994) (end 115.525 61.811994) (width 0.3) (layer F.Cu) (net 13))
 (segment (start 115.525 61.811994) (end 121.285 67.571994) (width 0.3) (layer F.Cu) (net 13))
 (segment (start 115.151994 63.081994) (end 112.84 63.081994) (width 0.3) (layer F.Cu) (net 14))
 (segment (start 121.031 68.961) (end 115.151994 63.081994) (width 0.3) (layer F.Cu) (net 14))
 (segment (start 131.445 67.571994) (end 130.055994 68.961) (width 0.3) (layer F.Cu) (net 14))
 (segment (start 130.055994 68.961) (end 121.031 68.961) (width 0.3) (layer F.Cu) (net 14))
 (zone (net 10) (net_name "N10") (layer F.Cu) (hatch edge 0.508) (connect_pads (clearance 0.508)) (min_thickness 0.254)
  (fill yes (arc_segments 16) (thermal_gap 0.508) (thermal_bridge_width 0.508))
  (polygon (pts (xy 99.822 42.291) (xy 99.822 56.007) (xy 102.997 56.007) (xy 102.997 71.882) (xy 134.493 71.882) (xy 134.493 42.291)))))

